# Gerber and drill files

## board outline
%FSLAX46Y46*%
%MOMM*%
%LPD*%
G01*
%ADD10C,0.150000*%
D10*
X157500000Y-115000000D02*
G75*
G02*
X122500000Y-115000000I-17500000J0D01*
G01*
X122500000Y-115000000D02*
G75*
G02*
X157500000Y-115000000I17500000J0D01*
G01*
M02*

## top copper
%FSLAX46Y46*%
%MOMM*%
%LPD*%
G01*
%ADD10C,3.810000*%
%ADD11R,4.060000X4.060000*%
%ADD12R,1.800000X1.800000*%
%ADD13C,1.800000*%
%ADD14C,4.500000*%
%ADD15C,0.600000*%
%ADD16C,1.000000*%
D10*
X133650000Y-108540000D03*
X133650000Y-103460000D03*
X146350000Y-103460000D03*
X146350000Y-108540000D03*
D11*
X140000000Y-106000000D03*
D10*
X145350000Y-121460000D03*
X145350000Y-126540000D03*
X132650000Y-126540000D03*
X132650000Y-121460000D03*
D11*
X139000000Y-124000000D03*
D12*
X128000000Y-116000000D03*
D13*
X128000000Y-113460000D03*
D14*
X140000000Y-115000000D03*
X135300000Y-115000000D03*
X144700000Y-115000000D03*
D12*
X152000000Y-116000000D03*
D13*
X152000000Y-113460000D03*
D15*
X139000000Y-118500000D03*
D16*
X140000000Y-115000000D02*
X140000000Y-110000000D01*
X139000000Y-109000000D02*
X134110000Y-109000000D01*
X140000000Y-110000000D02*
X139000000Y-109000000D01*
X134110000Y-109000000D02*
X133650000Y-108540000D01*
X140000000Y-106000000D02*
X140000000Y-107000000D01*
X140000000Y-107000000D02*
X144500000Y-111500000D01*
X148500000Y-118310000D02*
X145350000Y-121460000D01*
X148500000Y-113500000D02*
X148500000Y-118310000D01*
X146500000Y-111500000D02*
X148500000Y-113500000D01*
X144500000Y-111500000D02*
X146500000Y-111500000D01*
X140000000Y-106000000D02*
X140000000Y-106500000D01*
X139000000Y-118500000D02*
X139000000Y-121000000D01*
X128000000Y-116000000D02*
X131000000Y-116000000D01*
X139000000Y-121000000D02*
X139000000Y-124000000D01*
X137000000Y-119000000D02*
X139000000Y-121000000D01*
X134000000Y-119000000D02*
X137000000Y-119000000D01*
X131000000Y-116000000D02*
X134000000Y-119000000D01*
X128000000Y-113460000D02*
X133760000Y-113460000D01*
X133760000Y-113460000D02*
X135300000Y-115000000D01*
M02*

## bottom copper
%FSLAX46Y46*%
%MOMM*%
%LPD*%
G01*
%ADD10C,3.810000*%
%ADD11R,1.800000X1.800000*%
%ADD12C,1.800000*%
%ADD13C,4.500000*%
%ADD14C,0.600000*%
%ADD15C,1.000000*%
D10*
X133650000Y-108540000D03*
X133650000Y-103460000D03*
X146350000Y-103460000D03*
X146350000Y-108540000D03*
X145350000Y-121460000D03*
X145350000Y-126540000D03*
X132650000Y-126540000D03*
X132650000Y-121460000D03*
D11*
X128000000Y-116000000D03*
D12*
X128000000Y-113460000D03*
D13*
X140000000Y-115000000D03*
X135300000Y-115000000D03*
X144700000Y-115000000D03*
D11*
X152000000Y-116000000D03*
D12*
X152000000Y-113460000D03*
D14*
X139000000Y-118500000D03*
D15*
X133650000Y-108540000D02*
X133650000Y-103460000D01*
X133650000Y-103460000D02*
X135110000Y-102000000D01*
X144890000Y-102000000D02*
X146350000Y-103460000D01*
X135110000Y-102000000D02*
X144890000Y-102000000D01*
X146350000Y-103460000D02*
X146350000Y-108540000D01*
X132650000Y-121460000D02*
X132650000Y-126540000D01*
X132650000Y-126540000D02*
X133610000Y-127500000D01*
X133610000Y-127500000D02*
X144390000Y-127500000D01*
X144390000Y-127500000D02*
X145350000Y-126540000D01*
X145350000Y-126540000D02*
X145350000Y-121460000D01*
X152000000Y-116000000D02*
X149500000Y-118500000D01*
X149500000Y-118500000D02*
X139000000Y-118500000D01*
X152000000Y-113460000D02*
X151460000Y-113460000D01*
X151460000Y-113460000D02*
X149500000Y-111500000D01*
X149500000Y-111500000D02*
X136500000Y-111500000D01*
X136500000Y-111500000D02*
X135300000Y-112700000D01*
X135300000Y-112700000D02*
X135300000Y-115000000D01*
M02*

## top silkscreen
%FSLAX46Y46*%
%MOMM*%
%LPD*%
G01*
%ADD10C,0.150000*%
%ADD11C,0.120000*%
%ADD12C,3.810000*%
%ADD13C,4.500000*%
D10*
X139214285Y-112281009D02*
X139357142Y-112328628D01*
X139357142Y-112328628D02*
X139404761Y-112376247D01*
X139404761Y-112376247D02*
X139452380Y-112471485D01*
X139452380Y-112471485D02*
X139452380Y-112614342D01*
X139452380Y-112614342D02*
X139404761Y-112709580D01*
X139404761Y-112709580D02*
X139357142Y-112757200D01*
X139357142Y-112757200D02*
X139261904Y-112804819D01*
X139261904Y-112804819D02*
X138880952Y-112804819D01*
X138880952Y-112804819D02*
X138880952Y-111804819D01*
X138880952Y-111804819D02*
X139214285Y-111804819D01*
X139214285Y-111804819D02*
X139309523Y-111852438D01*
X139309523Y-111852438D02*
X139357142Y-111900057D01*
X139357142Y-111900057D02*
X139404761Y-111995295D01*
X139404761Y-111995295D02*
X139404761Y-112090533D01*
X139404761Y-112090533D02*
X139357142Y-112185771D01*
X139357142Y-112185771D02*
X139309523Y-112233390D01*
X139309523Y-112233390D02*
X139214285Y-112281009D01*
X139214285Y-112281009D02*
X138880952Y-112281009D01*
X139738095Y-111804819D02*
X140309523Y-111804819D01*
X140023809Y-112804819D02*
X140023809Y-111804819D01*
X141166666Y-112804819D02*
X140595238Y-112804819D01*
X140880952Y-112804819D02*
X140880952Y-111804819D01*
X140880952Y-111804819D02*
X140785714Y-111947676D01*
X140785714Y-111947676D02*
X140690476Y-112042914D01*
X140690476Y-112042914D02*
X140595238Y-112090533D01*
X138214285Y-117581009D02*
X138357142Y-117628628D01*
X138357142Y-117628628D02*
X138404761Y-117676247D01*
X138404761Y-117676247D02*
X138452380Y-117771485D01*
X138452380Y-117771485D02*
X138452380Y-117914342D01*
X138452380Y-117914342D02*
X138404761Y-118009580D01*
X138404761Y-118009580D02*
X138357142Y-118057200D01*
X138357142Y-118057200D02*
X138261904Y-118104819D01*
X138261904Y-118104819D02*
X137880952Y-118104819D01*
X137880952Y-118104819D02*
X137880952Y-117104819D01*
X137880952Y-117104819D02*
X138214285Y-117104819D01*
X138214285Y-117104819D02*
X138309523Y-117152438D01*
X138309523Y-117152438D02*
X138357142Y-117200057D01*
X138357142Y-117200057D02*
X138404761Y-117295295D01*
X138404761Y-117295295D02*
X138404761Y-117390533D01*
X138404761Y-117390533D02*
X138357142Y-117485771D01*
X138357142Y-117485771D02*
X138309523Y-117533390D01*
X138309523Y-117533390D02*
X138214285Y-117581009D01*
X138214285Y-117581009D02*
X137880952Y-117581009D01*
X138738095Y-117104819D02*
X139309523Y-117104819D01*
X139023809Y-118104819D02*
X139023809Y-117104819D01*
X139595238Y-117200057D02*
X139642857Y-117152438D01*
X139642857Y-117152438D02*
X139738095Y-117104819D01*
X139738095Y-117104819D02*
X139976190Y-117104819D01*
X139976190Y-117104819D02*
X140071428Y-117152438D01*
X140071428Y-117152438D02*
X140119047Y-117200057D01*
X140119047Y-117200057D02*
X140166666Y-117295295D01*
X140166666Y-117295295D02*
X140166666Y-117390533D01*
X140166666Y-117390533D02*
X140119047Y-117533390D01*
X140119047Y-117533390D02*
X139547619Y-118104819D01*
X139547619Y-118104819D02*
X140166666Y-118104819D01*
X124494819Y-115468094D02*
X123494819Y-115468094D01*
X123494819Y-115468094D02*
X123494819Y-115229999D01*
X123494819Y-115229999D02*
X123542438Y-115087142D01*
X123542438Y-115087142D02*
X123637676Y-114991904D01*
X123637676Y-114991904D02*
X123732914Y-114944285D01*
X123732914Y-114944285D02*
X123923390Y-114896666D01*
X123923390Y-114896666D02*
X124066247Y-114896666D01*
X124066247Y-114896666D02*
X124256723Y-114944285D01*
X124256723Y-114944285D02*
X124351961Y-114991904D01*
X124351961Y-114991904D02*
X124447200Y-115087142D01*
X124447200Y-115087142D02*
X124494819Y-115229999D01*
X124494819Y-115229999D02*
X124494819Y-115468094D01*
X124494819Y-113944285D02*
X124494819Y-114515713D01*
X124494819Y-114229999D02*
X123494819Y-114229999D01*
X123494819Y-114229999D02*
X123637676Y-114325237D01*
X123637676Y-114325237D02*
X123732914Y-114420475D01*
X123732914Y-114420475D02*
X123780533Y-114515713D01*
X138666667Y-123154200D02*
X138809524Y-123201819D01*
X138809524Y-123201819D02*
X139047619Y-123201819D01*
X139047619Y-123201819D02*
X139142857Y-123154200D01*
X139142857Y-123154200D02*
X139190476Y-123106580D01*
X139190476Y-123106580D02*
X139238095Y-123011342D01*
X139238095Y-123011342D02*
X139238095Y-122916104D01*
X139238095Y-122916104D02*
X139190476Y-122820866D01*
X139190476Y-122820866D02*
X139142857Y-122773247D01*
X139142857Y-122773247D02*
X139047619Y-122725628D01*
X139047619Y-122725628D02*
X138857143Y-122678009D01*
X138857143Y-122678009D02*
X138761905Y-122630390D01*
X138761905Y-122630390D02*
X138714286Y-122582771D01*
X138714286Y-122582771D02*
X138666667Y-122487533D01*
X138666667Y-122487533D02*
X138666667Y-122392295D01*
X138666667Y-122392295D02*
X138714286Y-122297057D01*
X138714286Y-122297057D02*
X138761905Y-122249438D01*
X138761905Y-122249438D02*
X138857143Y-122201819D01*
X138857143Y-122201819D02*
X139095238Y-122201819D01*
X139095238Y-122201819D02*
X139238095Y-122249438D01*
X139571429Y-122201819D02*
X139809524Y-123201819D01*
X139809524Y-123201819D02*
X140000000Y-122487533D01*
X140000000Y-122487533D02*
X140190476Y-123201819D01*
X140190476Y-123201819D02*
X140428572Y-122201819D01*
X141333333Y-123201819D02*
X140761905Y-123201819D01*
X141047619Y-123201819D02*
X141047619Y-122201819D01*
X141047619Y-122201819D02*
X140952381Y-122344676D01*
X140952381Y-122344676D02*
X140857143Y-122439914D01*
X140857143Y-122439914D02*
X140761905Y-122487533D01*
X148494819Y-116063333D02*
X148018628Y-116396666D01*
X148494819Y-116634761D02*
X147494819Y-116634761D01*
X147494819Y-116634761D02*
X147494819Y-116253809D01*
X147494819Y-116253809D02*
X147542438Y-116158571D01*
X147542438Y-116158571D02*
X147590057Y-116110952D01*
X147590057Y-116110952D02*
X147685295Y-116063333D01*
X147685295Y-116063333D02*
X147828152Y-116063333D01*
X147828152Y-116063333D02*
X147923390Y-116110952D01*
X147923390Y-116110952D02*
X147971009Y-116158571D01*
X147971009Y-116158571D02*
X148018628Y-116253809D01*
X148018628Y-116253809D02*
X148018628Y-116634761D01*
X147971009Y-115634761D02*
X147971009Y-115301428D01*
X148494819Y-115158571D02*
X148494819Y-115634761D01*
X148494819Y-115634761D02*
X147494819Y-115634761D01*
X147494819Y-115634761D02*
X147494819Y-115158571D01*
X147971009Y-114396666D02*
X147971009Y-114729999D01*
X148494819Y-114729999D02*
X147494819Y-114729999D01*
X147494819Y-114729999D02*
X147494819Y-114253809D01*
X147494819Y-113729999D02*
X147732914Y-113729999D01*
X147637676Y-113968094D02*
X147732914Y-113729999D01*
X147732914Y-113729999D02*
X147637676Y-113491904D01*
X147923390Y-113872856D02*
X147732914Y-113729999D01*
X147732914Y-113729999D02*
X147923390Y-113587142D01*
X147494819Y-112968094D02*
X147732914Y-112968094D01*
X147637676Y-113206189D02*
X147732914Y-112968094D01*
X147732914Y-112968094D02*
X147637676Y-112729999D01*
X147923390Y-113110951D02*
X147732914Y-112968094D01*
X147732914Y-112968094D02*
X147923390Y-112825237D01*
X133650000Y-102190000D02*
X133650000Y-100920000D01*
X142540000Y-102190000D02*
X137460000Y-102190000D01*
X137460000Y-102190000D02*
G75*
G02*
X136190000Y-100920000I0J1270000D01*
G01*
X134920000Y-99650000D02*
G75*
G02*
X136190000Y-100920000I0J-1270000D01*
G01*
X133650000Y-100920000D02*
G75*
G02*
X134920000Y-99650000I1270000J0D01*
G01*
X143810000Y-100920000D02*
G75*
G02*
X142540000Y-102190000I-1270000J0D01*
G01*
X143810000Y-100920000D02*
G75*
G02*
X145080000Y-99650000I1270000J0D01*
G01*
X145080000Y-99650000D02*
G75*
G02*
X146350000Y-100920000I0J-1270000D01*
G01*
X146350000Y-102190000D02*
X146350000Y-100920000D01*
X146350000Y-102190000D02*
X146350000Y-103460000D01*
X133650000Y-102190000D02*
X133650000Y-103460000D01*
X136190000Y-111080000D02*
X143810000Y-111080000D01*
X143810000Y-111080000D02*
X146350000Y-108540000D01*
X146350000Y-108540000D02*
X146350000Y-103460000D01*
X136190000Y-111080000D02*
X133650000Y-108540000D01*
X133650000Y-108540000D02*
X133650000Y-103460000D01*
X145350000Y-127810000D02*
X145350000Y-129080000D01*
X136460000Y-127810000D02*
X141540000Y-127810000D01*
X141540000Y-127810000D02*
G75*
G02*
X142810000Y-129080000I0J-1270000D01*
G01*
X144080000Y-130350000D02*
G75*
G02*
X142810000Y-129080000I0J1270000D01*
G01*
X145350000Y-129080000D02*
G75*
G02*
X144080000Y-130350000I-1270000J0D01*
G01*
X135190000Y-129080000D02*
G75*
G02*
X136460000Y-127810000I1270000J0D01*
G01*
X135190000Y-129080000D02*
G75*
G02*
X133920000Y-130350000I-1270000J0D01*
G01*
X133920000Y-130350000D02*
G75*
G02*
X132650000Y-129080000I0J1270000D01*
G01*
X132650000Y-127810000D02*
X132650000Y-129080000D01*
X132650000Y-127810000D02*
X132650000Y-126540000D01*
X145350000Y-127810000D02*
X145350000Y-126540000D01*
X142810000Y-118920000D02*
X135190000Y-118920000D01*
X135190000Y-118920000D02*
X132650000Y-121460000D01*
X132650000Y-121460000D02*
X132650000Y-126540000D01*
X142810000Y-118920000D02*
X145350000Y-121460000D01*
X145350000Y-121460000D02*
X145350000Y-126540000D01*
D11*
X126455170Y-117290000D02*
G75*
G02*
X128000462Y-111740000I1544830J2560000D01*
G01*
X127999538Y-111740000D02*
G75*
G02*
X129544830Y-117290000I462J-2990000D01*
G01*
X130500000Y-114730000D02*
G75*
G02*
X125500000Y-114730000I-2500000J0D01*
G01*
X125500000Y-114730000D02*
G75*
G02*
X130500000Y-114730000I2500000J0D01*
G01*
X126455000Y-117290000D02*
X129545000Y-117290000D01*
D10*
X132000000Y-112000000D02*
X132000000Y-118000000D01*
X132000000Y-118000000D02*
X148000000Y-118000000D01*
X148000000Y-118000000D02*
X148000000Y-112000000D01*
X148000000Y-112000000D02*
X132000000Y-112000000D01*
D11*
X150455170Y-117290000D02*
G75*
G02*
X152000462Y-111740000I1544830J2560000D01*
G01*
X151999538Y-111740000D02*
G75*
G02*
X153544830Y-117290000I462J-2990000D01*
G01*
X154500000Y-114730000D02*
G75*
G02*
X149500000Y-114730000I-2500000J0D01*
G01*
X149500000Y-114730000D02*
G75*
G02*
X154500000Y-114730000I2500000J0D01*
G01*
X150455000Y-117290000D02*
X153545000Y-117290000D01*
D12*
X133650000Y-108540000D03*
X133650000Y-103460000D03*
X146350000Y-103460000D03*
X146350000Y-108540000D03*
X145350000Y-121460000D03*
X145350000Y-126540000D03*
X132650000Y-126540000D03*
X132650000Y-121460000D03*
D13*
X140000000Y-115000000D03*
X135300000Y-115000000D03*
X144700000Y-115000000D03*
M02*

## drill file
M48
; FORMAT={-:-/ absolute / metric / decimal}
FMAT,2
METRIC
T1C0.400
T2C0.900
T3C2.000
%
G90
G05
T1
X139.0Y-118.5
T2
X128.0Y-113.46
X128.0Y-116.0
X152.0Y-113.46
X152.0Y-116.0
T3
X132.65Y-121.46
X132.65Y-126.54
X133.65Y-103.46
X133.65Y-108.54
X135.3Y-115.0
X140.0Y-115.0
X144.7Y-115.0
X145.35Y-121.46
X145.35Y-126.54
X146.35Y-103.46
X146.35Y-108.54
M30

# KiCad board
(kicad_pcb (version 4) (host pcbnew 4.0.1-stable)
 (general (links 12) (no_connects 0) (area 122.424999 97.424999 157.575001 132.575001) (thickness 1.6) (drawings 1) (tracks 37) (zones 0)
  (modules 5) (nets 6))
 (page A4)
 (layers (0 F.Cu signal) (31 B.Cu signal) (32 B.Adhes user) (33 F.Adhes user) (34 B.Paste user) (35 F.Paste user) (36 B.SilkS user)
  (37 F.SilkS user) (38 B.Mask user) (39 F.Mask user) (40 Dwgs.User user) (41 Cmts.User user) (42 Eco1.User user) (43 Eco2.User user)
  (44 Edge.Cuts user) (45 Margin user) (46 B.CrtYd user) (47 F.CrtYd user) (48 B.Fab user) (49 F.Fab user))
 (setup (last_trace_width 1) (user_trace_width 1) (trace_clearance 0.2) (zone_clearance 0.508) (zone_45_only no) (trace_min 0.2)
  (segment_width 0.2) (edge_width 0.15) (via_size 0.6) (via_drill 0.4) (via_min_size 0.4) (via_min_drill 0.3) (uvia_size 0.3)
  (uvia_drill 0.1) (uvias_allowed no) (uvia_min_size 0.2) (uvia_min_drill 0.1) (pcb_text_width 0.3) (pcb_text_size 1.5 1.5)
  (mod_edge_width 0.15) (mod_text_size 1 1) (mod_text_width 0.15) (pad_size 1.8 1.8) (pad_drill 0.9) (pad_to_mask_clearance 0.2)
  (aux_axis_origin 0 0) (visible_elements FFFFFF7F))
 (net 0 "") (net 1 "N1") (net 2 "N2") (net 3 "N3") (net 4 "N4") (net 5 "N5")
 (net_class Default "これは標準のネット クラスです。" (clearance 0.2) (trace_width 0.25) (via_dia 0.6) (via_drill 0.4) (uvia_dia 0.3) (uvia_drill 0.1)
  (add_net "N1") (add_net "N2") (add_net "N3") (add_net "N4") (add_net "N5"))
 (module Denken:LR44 (layer F.Cu) (at 140 106)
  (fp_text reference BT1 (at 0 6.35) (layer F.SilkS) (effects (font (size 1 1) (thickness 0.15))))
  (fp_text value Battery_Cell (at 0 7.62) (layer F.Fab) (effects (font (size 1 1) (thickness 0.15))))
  (fp_line (start -6.35 -3.81) (end -6.35 -5.08) (layer F.SilkS) (width 0.15))
  (fp_line (start 2.54 -3.81) (end -2.54 -3.81) (layer F.SilkS) (width 0.15))
  (fp_arc (start -2.54 -5.08) (end -2.54 -3.81) (angle 90) (layer F.SilkS) (width 0.15))
  (fp_arc (start -5.08 -5.08) (end -5.08 -6.35) (angle 90) (layer F.SilkS) (width 0.15))
  (fp_arc (start -5.08 -5.08) (end -6.35 -5.08) (angle 90) (layer F.SilkS) (width 0.15))
  (fp_arc (start 2.54 -5.08) (end 3.81 -5.08) (angle 90) (layer F.SilkS) (width 0.15))
  (fp_arc (start 5.08 -5.08) (end 3.81 -5.08) (angle 90) (layer F.SilkS) (width 0.15))
  (fp_arc (start 5.08 -5.08) (end 5.08 -6.35) (angle 90) (layer F.SilkS) (width 0.15))
  (fp_line (start 6.35 -3.81) (end 6.35 -5.08) (layer F.SilkS) (width 0.15))
  (fp_line (start 6.35 -3.81) (end 6.35 -2.54) (layer F.SilkS) (width 0.15))
  (fp_line (start -6.35 -3.81) (end -6.35 -2.54) (layer F.SilkS) (width 0.15))
  (fp_line (start -3.81 5.08) (end 3.81 5.08) (layer F.SilkS) (width 0.15))
  (fp_line (start 3.81 5.08) (end 6.35 2.54) (layer F.SilkS) (width 0.15))
  (fp_line (start 6.35 2.54) (end 6.35 -2.54) (layer F.SilkS) (width 0.15))
  (fp_line (start -3.81 5.08) (end -6.35 2.54) (layer F.SilkS) (width 0.15))
  (fp_line (start -6.35 2.54) (end -6.35 -2.54) (layer F.SilkS) (width 0.15))
  (pad 1 thru_hole circle (at -6.35 2.54) (size 3.81 3.81) (drill 2) (layers *.Cu *.Mask F.SilkS) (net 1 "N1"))
  (pad 1 thru_hole circle (at -6.35 -2.54) (size 3.81 3.81) (drill 2) (layers *.Cu *.Mask F.SilkS) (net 1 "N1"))
  (pad 1 thru_hole circle (at 6.35 -2.54) (size 3.81 3.81) (drill 2) (layers *.Cu *.Mask F.SilkS) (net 1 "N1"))
  (pad 1 thru_hole circle (at 6.35 2.54) (size 3.81 3.81) (drill 2) (layers *.Cu *.Mask F.SilkS) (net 1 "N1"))
  (pad 2 smd rect (at 0 0) (size 4.06 4.06) (layers F.Cu F.Paste F.Mask) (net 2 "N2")))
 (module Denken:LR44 (layer F.Cu) (at 139 124 180)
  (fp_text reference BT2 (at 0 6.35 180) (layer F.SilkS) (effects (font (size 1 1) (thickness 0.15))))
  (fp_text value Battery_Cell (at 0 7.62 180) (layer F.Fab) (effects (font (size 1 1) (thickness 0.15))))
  (fp_line (start -6.35 -3.81) (end -6.35 -5.08) (layer F.SilkS) (width 0.15))
  (fp_line (start 2.54 -3.81) (end -2.54 -3.81) (layer F.SilkS) (width 0.15))
  (fp_arc (start -2.54 -5.08) (end -2.54 -3.81) (angle 90) (layer F.SilkS) (width 0.15))
  (fp_arc (start -5.08 -5.08) (end -5.08 -6.35) (angle 90) (layer F.SilkS) (width 0.15))
  (fp_arc (start -5.08 -5.08) (end -6.35 -5.08) (angle 90) (layer F.SilkS) (width 0.15))
  (fp_arc (start 2.54 -5.08) (end 3.81 -5.08) (angle 90) (layer F.SilkS) (width 0.15))
  (fp_arc (start 5.08 -5.08) (end 3.81 -5.08) (angle 90) (layer F.SilkS) (width 0.15))
  (fp_arc (start 5.08 -5.08) (end 5.08 -6.35) (angle 90) (layer F.SilkS) (width 0.15))
  (fp_line (start 6.35 -3.81) (end 6.35 -5.08) (layer F.SilkS) (width 0.15))
  (fp_line (start 6.35 -3.81) (end 6.35 -2.54) (layer F.SilkS) (width 0.15))
  (fp_line (start -6.35 -3.81) (end -6.35 -2.54) (layer F.SilkS) (width 0.15))
  (fp_line (start -3.81 5.08) (end 3.81 5.08) (layer F.SilkS) (width 0.15))
  (fp_line (start 3.81 5.08) (end 6.35 2.54) (layer F.SilkS) (width 0.15))
  (fp_line (start 6.35 2.54) (end 6.35 -2.54) (layer F.SilkS) (width 0.15))
  (fp_line (start -3.81 5.08) (end -6.35 2.54) (layer F.SilkS) (width 0.15))
  (fp_line (start -6.35 2.54) (end -6.35 -2.54) (layer F.SilkS) (width 0.15))
  (pad 1 thru_hole circle (at -6.35 2.54 180) (size 3.81 3.81) (drill 2) (layers *.Cu *.Mask F.SilkS) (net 2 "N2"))
  (pad 1 thru_hole circle (at -6.35 -2.54 180) (size 3.81 3.81) (drill 2) (layers *.Cu *.Mask F.SilkS) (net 2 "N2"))
  (pad 1 thru_hole circle (at 6.35 -2.54 180) (size 3.81 3.81) (drill 2) (layers *.Cu *.Mask F.SilkS) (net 2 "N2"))
  (pad 1 thru_hole circle (at 6.35 2.54 180) (size 3.81 3.81) (drill 2) (layers *.Cu *.Mask F.SilkS) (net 2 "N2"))
  (pad 2 smd rect (at 0 0 180) (size 4.06 4.06) (layers F.Cu F.Paste F.Mask) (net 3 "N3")))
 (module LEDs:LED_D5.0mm (layer F.Cu) (at 128 116 90)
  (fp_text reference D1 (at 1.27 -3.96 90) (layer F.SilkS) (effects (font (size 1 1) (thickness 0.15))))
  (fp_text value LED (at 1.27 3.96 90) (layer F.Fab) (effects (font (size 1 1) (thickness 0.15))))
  (fp_arc (start 1.27 0) (end -1.29 -1.54483) (angle 148.9) (layer F.SilkS) (width 0.12))
  (fp_arc (start 1.27 0) (end -1.29 1.54483) (angle -148.9) (layer F.SilkS) (width 0.12))
  (fp_circle (center 1.27 0) (end 3.77 0) (layer F.SilkS) (width 0.12))
  (fp_line (start -1.29 -1.545) (end -1.29 1.545) (layer F.SilkS) (width 0.12))
  (pad 1 thru_hole rect (at 0 0 90) (size 1.8 1.8) (drill 0.9) (layers *.Cu *.Mask) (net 3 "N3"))
  (pad 2 thru_hole circle (at 2.54 0 90) (size 1.8 1.8) (drill 0.9) (layers *.Cu *.Mask) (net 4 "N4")))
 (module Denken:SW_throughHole (layer F.Cu) (at 140 115)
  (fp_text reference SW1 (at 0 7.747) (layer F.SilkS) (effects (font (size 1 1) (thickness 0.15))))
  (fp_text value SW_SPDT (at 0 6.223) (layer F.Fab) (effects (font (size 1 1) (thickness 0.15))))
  (fp_line (start -8 -3) (end -8 3) (layer F.SilkS) (width 0.15))
  (fp_line (start -8 3) (end 8 3) (layer F.SilkS) (width 0.15))
  (fp_line (start 8 3) (end 8 -3) (layer F.SilkS) (width 0.15))
  (fp_line (start 8 -3) (end -8 -3) (layer F.SilkS) (width 0.15))
  (pad 2 thru_hole circle (at 0 0) (size 4.5 4.5) (drill 2) (layers *.Cu *.Mask F.SilkS) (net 1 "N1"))
  (pad 1 thru_hole circle (at -4.7 0) (size 4.5 4.5) (drill 2) (layers *.Cu *.Mask F.SilkS) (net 4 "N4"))
  (pad 3 thru_hole circle (at 4.7 0) (size 4.5 4.5) (drill 2) (layers *.Cu *.Mask F.SilkS) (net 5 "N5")))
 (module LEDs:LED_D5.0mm (layer F.Cu) (at 152 116 90)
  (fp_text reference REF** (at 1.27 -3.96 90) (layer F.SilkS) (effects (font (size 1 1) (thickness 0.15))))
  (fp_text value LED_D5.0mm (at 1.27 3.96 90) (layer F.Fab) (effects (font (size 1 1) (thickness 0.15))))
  (fp_arc (start 1.27 0) (end -1.29 -1.54483) (angle 148.9) (layer F.SilkS) (width 0.12))
  (fp_arc (start 1.27 0) (end -1.29 1.54483) (angle -148.9) (layer F.SilkS) (width 0.12))
  (fp_circle (center 1.27 0) (end 3.77 0) (layer F.SilkS) (width 0.12))
  (fp_line (start -1.29 -1.545) (end -1.29 1.545) (layer F.SilkS) (width 0.12))
  (pad 1 thru_hole rect (at 0 0 90) (size 1.8 1.8) (drill 0.9) (layers *.Cu *.Mask) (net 3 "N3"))
  (pad 2 thru_hole circle (at 2.54 0 90) (size 1.8 1.8) (drill 0.9) (layers *.Cu *.Mask) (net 4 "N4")))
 (gr_circle (center 140 115) (end 157.5 115) (layer Edge.Cuts) (width 0.15))
 (segment (start 133.65 108.54) (end 133.65 103.46) (width 1) (layer B.Cu) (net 1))
 (segment (start 133.65 103.46) (end 135.11 102) (width 1) (layer B.Cu) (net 1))
 (segment (start 144.89 102) (end 146.35 103.46) (width 1) (layer B.Cu) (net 1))
 (segment (start 135.11 102) (end 144.89 102) (width 1) (layer B.Cu) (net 1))
 (segment (start 146.35 103.46) (end 146.35 108.54) (width 1) (layer B.Cu) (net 1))
 (segment (start 140 115) (end 140 110) (width 1) (layer F.Cu) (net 1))
 (segment (start 139 109) (end 134.11 109) (width 1) (layer F.Cu) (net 1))
 (segment (start 140 110) (end 139 109) (width 1) (layer F.Cu) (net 1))
 (segment (start 134.11 109) (end 133.65 108.54) (width 1) (layer F.Cu) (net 1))
 (segment (start 140 106) (end 140 107) (width 1) (layer F.Cu) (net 2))
 (segment (start 140 107) (end 144.5 111.5) (width 1) (layer F.Cu) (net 2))
 (segment (start 148.5 118.31) (end 145.35 121.46) (width 1) (layer F.Cu) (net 2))
 (segment (start 148.5 113.5) (end 148.5 118.31) (width 1) (layer F.Cu) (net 2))
 (segment (start 146.5 111.5) (end 148.5 113.5) (width 1) (layer F.Cu) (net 2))
 (segment (start 144.5 111.5) (end 146.5 111.5) (width 1) (layer F.Cu) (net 2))
 (segment (start 132.65 121.46) (end 132.65 126.54) (width 1) (layer B.Cu) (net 2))
 (segment (start 132.65 126.54) (end 133.61 127.5) (width 1) (layer B.Cu) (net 2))
 (segment (start 133.61 127.5) (end 144.39 127.5) (width 1) (layer B.Cu) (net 2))
 (segment (start 144.39 127.5) (end 145.35 126.54) (width 1) (layer B.Cu) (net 2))
 (segment (start 145.35 126.54) (end 145.35 121.46) (width 1) (layer B.Cu) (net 2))
 (segment (start 140 106) (end 140 106.5) (width 1) (layer F.Cu) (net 2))
 (segment (start 152 116) (end 149.5 118.5) (width 1) (layer B.Cu) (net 3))
 (segment (start 139 118.5) (end 139 121) (width 1) (layer F.Cu) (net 3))
 (via (at 139 118.5) (size 0.6) (drill 0.4) (layers F.Cu B.Cu) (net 3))
 (segment (start 149.5 118.5) (end 139 118.5) (width 1) (layer B.Cu) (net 3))
 (segment (start 128 116) (end 131 116) (width 1) (layer F.Cu) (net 3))
 (segment (start 139 121) (end 139 124) (width 1) (layer F.Cu) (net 3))
 (segment (start 137 119) (end 139 121) (width 1) (layer F.Cu) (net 3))
 (segment (start 134 119) (end 137 119) (width 1) (layer F.Cu) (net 3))
 (segment (start 131 116) (end 134 119) (width 1) (layer F.Cu) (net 3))
 (segment (start 152 113.46) (end 151.46 113.46) (width 1) (layer B.Cu) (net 4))
 (segment (start 151.46 113.46) (end 149.5 111.5) (width 1) (layer B.Cu) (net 4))
 (segment (start 149.5 111.5) (end 136.5 111.5) (width 1) (layer B.Cu) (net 4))
 (segment (start 136.5 111.5) (end 135.3 112.7) (width 1) (layer B.Cu) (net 4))
 (segment (start 135.3 112.7) (end 135.3 115) (width 1) (layer B.Cu) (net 4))
 (segment (start 128 113.46) (end 133.76 113.46) (width 1) (layer F.Cu) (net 4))
 (segment (start 133.76 113.46) (end 135.3 115) (width 1) (layer F.Cu) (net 4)))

